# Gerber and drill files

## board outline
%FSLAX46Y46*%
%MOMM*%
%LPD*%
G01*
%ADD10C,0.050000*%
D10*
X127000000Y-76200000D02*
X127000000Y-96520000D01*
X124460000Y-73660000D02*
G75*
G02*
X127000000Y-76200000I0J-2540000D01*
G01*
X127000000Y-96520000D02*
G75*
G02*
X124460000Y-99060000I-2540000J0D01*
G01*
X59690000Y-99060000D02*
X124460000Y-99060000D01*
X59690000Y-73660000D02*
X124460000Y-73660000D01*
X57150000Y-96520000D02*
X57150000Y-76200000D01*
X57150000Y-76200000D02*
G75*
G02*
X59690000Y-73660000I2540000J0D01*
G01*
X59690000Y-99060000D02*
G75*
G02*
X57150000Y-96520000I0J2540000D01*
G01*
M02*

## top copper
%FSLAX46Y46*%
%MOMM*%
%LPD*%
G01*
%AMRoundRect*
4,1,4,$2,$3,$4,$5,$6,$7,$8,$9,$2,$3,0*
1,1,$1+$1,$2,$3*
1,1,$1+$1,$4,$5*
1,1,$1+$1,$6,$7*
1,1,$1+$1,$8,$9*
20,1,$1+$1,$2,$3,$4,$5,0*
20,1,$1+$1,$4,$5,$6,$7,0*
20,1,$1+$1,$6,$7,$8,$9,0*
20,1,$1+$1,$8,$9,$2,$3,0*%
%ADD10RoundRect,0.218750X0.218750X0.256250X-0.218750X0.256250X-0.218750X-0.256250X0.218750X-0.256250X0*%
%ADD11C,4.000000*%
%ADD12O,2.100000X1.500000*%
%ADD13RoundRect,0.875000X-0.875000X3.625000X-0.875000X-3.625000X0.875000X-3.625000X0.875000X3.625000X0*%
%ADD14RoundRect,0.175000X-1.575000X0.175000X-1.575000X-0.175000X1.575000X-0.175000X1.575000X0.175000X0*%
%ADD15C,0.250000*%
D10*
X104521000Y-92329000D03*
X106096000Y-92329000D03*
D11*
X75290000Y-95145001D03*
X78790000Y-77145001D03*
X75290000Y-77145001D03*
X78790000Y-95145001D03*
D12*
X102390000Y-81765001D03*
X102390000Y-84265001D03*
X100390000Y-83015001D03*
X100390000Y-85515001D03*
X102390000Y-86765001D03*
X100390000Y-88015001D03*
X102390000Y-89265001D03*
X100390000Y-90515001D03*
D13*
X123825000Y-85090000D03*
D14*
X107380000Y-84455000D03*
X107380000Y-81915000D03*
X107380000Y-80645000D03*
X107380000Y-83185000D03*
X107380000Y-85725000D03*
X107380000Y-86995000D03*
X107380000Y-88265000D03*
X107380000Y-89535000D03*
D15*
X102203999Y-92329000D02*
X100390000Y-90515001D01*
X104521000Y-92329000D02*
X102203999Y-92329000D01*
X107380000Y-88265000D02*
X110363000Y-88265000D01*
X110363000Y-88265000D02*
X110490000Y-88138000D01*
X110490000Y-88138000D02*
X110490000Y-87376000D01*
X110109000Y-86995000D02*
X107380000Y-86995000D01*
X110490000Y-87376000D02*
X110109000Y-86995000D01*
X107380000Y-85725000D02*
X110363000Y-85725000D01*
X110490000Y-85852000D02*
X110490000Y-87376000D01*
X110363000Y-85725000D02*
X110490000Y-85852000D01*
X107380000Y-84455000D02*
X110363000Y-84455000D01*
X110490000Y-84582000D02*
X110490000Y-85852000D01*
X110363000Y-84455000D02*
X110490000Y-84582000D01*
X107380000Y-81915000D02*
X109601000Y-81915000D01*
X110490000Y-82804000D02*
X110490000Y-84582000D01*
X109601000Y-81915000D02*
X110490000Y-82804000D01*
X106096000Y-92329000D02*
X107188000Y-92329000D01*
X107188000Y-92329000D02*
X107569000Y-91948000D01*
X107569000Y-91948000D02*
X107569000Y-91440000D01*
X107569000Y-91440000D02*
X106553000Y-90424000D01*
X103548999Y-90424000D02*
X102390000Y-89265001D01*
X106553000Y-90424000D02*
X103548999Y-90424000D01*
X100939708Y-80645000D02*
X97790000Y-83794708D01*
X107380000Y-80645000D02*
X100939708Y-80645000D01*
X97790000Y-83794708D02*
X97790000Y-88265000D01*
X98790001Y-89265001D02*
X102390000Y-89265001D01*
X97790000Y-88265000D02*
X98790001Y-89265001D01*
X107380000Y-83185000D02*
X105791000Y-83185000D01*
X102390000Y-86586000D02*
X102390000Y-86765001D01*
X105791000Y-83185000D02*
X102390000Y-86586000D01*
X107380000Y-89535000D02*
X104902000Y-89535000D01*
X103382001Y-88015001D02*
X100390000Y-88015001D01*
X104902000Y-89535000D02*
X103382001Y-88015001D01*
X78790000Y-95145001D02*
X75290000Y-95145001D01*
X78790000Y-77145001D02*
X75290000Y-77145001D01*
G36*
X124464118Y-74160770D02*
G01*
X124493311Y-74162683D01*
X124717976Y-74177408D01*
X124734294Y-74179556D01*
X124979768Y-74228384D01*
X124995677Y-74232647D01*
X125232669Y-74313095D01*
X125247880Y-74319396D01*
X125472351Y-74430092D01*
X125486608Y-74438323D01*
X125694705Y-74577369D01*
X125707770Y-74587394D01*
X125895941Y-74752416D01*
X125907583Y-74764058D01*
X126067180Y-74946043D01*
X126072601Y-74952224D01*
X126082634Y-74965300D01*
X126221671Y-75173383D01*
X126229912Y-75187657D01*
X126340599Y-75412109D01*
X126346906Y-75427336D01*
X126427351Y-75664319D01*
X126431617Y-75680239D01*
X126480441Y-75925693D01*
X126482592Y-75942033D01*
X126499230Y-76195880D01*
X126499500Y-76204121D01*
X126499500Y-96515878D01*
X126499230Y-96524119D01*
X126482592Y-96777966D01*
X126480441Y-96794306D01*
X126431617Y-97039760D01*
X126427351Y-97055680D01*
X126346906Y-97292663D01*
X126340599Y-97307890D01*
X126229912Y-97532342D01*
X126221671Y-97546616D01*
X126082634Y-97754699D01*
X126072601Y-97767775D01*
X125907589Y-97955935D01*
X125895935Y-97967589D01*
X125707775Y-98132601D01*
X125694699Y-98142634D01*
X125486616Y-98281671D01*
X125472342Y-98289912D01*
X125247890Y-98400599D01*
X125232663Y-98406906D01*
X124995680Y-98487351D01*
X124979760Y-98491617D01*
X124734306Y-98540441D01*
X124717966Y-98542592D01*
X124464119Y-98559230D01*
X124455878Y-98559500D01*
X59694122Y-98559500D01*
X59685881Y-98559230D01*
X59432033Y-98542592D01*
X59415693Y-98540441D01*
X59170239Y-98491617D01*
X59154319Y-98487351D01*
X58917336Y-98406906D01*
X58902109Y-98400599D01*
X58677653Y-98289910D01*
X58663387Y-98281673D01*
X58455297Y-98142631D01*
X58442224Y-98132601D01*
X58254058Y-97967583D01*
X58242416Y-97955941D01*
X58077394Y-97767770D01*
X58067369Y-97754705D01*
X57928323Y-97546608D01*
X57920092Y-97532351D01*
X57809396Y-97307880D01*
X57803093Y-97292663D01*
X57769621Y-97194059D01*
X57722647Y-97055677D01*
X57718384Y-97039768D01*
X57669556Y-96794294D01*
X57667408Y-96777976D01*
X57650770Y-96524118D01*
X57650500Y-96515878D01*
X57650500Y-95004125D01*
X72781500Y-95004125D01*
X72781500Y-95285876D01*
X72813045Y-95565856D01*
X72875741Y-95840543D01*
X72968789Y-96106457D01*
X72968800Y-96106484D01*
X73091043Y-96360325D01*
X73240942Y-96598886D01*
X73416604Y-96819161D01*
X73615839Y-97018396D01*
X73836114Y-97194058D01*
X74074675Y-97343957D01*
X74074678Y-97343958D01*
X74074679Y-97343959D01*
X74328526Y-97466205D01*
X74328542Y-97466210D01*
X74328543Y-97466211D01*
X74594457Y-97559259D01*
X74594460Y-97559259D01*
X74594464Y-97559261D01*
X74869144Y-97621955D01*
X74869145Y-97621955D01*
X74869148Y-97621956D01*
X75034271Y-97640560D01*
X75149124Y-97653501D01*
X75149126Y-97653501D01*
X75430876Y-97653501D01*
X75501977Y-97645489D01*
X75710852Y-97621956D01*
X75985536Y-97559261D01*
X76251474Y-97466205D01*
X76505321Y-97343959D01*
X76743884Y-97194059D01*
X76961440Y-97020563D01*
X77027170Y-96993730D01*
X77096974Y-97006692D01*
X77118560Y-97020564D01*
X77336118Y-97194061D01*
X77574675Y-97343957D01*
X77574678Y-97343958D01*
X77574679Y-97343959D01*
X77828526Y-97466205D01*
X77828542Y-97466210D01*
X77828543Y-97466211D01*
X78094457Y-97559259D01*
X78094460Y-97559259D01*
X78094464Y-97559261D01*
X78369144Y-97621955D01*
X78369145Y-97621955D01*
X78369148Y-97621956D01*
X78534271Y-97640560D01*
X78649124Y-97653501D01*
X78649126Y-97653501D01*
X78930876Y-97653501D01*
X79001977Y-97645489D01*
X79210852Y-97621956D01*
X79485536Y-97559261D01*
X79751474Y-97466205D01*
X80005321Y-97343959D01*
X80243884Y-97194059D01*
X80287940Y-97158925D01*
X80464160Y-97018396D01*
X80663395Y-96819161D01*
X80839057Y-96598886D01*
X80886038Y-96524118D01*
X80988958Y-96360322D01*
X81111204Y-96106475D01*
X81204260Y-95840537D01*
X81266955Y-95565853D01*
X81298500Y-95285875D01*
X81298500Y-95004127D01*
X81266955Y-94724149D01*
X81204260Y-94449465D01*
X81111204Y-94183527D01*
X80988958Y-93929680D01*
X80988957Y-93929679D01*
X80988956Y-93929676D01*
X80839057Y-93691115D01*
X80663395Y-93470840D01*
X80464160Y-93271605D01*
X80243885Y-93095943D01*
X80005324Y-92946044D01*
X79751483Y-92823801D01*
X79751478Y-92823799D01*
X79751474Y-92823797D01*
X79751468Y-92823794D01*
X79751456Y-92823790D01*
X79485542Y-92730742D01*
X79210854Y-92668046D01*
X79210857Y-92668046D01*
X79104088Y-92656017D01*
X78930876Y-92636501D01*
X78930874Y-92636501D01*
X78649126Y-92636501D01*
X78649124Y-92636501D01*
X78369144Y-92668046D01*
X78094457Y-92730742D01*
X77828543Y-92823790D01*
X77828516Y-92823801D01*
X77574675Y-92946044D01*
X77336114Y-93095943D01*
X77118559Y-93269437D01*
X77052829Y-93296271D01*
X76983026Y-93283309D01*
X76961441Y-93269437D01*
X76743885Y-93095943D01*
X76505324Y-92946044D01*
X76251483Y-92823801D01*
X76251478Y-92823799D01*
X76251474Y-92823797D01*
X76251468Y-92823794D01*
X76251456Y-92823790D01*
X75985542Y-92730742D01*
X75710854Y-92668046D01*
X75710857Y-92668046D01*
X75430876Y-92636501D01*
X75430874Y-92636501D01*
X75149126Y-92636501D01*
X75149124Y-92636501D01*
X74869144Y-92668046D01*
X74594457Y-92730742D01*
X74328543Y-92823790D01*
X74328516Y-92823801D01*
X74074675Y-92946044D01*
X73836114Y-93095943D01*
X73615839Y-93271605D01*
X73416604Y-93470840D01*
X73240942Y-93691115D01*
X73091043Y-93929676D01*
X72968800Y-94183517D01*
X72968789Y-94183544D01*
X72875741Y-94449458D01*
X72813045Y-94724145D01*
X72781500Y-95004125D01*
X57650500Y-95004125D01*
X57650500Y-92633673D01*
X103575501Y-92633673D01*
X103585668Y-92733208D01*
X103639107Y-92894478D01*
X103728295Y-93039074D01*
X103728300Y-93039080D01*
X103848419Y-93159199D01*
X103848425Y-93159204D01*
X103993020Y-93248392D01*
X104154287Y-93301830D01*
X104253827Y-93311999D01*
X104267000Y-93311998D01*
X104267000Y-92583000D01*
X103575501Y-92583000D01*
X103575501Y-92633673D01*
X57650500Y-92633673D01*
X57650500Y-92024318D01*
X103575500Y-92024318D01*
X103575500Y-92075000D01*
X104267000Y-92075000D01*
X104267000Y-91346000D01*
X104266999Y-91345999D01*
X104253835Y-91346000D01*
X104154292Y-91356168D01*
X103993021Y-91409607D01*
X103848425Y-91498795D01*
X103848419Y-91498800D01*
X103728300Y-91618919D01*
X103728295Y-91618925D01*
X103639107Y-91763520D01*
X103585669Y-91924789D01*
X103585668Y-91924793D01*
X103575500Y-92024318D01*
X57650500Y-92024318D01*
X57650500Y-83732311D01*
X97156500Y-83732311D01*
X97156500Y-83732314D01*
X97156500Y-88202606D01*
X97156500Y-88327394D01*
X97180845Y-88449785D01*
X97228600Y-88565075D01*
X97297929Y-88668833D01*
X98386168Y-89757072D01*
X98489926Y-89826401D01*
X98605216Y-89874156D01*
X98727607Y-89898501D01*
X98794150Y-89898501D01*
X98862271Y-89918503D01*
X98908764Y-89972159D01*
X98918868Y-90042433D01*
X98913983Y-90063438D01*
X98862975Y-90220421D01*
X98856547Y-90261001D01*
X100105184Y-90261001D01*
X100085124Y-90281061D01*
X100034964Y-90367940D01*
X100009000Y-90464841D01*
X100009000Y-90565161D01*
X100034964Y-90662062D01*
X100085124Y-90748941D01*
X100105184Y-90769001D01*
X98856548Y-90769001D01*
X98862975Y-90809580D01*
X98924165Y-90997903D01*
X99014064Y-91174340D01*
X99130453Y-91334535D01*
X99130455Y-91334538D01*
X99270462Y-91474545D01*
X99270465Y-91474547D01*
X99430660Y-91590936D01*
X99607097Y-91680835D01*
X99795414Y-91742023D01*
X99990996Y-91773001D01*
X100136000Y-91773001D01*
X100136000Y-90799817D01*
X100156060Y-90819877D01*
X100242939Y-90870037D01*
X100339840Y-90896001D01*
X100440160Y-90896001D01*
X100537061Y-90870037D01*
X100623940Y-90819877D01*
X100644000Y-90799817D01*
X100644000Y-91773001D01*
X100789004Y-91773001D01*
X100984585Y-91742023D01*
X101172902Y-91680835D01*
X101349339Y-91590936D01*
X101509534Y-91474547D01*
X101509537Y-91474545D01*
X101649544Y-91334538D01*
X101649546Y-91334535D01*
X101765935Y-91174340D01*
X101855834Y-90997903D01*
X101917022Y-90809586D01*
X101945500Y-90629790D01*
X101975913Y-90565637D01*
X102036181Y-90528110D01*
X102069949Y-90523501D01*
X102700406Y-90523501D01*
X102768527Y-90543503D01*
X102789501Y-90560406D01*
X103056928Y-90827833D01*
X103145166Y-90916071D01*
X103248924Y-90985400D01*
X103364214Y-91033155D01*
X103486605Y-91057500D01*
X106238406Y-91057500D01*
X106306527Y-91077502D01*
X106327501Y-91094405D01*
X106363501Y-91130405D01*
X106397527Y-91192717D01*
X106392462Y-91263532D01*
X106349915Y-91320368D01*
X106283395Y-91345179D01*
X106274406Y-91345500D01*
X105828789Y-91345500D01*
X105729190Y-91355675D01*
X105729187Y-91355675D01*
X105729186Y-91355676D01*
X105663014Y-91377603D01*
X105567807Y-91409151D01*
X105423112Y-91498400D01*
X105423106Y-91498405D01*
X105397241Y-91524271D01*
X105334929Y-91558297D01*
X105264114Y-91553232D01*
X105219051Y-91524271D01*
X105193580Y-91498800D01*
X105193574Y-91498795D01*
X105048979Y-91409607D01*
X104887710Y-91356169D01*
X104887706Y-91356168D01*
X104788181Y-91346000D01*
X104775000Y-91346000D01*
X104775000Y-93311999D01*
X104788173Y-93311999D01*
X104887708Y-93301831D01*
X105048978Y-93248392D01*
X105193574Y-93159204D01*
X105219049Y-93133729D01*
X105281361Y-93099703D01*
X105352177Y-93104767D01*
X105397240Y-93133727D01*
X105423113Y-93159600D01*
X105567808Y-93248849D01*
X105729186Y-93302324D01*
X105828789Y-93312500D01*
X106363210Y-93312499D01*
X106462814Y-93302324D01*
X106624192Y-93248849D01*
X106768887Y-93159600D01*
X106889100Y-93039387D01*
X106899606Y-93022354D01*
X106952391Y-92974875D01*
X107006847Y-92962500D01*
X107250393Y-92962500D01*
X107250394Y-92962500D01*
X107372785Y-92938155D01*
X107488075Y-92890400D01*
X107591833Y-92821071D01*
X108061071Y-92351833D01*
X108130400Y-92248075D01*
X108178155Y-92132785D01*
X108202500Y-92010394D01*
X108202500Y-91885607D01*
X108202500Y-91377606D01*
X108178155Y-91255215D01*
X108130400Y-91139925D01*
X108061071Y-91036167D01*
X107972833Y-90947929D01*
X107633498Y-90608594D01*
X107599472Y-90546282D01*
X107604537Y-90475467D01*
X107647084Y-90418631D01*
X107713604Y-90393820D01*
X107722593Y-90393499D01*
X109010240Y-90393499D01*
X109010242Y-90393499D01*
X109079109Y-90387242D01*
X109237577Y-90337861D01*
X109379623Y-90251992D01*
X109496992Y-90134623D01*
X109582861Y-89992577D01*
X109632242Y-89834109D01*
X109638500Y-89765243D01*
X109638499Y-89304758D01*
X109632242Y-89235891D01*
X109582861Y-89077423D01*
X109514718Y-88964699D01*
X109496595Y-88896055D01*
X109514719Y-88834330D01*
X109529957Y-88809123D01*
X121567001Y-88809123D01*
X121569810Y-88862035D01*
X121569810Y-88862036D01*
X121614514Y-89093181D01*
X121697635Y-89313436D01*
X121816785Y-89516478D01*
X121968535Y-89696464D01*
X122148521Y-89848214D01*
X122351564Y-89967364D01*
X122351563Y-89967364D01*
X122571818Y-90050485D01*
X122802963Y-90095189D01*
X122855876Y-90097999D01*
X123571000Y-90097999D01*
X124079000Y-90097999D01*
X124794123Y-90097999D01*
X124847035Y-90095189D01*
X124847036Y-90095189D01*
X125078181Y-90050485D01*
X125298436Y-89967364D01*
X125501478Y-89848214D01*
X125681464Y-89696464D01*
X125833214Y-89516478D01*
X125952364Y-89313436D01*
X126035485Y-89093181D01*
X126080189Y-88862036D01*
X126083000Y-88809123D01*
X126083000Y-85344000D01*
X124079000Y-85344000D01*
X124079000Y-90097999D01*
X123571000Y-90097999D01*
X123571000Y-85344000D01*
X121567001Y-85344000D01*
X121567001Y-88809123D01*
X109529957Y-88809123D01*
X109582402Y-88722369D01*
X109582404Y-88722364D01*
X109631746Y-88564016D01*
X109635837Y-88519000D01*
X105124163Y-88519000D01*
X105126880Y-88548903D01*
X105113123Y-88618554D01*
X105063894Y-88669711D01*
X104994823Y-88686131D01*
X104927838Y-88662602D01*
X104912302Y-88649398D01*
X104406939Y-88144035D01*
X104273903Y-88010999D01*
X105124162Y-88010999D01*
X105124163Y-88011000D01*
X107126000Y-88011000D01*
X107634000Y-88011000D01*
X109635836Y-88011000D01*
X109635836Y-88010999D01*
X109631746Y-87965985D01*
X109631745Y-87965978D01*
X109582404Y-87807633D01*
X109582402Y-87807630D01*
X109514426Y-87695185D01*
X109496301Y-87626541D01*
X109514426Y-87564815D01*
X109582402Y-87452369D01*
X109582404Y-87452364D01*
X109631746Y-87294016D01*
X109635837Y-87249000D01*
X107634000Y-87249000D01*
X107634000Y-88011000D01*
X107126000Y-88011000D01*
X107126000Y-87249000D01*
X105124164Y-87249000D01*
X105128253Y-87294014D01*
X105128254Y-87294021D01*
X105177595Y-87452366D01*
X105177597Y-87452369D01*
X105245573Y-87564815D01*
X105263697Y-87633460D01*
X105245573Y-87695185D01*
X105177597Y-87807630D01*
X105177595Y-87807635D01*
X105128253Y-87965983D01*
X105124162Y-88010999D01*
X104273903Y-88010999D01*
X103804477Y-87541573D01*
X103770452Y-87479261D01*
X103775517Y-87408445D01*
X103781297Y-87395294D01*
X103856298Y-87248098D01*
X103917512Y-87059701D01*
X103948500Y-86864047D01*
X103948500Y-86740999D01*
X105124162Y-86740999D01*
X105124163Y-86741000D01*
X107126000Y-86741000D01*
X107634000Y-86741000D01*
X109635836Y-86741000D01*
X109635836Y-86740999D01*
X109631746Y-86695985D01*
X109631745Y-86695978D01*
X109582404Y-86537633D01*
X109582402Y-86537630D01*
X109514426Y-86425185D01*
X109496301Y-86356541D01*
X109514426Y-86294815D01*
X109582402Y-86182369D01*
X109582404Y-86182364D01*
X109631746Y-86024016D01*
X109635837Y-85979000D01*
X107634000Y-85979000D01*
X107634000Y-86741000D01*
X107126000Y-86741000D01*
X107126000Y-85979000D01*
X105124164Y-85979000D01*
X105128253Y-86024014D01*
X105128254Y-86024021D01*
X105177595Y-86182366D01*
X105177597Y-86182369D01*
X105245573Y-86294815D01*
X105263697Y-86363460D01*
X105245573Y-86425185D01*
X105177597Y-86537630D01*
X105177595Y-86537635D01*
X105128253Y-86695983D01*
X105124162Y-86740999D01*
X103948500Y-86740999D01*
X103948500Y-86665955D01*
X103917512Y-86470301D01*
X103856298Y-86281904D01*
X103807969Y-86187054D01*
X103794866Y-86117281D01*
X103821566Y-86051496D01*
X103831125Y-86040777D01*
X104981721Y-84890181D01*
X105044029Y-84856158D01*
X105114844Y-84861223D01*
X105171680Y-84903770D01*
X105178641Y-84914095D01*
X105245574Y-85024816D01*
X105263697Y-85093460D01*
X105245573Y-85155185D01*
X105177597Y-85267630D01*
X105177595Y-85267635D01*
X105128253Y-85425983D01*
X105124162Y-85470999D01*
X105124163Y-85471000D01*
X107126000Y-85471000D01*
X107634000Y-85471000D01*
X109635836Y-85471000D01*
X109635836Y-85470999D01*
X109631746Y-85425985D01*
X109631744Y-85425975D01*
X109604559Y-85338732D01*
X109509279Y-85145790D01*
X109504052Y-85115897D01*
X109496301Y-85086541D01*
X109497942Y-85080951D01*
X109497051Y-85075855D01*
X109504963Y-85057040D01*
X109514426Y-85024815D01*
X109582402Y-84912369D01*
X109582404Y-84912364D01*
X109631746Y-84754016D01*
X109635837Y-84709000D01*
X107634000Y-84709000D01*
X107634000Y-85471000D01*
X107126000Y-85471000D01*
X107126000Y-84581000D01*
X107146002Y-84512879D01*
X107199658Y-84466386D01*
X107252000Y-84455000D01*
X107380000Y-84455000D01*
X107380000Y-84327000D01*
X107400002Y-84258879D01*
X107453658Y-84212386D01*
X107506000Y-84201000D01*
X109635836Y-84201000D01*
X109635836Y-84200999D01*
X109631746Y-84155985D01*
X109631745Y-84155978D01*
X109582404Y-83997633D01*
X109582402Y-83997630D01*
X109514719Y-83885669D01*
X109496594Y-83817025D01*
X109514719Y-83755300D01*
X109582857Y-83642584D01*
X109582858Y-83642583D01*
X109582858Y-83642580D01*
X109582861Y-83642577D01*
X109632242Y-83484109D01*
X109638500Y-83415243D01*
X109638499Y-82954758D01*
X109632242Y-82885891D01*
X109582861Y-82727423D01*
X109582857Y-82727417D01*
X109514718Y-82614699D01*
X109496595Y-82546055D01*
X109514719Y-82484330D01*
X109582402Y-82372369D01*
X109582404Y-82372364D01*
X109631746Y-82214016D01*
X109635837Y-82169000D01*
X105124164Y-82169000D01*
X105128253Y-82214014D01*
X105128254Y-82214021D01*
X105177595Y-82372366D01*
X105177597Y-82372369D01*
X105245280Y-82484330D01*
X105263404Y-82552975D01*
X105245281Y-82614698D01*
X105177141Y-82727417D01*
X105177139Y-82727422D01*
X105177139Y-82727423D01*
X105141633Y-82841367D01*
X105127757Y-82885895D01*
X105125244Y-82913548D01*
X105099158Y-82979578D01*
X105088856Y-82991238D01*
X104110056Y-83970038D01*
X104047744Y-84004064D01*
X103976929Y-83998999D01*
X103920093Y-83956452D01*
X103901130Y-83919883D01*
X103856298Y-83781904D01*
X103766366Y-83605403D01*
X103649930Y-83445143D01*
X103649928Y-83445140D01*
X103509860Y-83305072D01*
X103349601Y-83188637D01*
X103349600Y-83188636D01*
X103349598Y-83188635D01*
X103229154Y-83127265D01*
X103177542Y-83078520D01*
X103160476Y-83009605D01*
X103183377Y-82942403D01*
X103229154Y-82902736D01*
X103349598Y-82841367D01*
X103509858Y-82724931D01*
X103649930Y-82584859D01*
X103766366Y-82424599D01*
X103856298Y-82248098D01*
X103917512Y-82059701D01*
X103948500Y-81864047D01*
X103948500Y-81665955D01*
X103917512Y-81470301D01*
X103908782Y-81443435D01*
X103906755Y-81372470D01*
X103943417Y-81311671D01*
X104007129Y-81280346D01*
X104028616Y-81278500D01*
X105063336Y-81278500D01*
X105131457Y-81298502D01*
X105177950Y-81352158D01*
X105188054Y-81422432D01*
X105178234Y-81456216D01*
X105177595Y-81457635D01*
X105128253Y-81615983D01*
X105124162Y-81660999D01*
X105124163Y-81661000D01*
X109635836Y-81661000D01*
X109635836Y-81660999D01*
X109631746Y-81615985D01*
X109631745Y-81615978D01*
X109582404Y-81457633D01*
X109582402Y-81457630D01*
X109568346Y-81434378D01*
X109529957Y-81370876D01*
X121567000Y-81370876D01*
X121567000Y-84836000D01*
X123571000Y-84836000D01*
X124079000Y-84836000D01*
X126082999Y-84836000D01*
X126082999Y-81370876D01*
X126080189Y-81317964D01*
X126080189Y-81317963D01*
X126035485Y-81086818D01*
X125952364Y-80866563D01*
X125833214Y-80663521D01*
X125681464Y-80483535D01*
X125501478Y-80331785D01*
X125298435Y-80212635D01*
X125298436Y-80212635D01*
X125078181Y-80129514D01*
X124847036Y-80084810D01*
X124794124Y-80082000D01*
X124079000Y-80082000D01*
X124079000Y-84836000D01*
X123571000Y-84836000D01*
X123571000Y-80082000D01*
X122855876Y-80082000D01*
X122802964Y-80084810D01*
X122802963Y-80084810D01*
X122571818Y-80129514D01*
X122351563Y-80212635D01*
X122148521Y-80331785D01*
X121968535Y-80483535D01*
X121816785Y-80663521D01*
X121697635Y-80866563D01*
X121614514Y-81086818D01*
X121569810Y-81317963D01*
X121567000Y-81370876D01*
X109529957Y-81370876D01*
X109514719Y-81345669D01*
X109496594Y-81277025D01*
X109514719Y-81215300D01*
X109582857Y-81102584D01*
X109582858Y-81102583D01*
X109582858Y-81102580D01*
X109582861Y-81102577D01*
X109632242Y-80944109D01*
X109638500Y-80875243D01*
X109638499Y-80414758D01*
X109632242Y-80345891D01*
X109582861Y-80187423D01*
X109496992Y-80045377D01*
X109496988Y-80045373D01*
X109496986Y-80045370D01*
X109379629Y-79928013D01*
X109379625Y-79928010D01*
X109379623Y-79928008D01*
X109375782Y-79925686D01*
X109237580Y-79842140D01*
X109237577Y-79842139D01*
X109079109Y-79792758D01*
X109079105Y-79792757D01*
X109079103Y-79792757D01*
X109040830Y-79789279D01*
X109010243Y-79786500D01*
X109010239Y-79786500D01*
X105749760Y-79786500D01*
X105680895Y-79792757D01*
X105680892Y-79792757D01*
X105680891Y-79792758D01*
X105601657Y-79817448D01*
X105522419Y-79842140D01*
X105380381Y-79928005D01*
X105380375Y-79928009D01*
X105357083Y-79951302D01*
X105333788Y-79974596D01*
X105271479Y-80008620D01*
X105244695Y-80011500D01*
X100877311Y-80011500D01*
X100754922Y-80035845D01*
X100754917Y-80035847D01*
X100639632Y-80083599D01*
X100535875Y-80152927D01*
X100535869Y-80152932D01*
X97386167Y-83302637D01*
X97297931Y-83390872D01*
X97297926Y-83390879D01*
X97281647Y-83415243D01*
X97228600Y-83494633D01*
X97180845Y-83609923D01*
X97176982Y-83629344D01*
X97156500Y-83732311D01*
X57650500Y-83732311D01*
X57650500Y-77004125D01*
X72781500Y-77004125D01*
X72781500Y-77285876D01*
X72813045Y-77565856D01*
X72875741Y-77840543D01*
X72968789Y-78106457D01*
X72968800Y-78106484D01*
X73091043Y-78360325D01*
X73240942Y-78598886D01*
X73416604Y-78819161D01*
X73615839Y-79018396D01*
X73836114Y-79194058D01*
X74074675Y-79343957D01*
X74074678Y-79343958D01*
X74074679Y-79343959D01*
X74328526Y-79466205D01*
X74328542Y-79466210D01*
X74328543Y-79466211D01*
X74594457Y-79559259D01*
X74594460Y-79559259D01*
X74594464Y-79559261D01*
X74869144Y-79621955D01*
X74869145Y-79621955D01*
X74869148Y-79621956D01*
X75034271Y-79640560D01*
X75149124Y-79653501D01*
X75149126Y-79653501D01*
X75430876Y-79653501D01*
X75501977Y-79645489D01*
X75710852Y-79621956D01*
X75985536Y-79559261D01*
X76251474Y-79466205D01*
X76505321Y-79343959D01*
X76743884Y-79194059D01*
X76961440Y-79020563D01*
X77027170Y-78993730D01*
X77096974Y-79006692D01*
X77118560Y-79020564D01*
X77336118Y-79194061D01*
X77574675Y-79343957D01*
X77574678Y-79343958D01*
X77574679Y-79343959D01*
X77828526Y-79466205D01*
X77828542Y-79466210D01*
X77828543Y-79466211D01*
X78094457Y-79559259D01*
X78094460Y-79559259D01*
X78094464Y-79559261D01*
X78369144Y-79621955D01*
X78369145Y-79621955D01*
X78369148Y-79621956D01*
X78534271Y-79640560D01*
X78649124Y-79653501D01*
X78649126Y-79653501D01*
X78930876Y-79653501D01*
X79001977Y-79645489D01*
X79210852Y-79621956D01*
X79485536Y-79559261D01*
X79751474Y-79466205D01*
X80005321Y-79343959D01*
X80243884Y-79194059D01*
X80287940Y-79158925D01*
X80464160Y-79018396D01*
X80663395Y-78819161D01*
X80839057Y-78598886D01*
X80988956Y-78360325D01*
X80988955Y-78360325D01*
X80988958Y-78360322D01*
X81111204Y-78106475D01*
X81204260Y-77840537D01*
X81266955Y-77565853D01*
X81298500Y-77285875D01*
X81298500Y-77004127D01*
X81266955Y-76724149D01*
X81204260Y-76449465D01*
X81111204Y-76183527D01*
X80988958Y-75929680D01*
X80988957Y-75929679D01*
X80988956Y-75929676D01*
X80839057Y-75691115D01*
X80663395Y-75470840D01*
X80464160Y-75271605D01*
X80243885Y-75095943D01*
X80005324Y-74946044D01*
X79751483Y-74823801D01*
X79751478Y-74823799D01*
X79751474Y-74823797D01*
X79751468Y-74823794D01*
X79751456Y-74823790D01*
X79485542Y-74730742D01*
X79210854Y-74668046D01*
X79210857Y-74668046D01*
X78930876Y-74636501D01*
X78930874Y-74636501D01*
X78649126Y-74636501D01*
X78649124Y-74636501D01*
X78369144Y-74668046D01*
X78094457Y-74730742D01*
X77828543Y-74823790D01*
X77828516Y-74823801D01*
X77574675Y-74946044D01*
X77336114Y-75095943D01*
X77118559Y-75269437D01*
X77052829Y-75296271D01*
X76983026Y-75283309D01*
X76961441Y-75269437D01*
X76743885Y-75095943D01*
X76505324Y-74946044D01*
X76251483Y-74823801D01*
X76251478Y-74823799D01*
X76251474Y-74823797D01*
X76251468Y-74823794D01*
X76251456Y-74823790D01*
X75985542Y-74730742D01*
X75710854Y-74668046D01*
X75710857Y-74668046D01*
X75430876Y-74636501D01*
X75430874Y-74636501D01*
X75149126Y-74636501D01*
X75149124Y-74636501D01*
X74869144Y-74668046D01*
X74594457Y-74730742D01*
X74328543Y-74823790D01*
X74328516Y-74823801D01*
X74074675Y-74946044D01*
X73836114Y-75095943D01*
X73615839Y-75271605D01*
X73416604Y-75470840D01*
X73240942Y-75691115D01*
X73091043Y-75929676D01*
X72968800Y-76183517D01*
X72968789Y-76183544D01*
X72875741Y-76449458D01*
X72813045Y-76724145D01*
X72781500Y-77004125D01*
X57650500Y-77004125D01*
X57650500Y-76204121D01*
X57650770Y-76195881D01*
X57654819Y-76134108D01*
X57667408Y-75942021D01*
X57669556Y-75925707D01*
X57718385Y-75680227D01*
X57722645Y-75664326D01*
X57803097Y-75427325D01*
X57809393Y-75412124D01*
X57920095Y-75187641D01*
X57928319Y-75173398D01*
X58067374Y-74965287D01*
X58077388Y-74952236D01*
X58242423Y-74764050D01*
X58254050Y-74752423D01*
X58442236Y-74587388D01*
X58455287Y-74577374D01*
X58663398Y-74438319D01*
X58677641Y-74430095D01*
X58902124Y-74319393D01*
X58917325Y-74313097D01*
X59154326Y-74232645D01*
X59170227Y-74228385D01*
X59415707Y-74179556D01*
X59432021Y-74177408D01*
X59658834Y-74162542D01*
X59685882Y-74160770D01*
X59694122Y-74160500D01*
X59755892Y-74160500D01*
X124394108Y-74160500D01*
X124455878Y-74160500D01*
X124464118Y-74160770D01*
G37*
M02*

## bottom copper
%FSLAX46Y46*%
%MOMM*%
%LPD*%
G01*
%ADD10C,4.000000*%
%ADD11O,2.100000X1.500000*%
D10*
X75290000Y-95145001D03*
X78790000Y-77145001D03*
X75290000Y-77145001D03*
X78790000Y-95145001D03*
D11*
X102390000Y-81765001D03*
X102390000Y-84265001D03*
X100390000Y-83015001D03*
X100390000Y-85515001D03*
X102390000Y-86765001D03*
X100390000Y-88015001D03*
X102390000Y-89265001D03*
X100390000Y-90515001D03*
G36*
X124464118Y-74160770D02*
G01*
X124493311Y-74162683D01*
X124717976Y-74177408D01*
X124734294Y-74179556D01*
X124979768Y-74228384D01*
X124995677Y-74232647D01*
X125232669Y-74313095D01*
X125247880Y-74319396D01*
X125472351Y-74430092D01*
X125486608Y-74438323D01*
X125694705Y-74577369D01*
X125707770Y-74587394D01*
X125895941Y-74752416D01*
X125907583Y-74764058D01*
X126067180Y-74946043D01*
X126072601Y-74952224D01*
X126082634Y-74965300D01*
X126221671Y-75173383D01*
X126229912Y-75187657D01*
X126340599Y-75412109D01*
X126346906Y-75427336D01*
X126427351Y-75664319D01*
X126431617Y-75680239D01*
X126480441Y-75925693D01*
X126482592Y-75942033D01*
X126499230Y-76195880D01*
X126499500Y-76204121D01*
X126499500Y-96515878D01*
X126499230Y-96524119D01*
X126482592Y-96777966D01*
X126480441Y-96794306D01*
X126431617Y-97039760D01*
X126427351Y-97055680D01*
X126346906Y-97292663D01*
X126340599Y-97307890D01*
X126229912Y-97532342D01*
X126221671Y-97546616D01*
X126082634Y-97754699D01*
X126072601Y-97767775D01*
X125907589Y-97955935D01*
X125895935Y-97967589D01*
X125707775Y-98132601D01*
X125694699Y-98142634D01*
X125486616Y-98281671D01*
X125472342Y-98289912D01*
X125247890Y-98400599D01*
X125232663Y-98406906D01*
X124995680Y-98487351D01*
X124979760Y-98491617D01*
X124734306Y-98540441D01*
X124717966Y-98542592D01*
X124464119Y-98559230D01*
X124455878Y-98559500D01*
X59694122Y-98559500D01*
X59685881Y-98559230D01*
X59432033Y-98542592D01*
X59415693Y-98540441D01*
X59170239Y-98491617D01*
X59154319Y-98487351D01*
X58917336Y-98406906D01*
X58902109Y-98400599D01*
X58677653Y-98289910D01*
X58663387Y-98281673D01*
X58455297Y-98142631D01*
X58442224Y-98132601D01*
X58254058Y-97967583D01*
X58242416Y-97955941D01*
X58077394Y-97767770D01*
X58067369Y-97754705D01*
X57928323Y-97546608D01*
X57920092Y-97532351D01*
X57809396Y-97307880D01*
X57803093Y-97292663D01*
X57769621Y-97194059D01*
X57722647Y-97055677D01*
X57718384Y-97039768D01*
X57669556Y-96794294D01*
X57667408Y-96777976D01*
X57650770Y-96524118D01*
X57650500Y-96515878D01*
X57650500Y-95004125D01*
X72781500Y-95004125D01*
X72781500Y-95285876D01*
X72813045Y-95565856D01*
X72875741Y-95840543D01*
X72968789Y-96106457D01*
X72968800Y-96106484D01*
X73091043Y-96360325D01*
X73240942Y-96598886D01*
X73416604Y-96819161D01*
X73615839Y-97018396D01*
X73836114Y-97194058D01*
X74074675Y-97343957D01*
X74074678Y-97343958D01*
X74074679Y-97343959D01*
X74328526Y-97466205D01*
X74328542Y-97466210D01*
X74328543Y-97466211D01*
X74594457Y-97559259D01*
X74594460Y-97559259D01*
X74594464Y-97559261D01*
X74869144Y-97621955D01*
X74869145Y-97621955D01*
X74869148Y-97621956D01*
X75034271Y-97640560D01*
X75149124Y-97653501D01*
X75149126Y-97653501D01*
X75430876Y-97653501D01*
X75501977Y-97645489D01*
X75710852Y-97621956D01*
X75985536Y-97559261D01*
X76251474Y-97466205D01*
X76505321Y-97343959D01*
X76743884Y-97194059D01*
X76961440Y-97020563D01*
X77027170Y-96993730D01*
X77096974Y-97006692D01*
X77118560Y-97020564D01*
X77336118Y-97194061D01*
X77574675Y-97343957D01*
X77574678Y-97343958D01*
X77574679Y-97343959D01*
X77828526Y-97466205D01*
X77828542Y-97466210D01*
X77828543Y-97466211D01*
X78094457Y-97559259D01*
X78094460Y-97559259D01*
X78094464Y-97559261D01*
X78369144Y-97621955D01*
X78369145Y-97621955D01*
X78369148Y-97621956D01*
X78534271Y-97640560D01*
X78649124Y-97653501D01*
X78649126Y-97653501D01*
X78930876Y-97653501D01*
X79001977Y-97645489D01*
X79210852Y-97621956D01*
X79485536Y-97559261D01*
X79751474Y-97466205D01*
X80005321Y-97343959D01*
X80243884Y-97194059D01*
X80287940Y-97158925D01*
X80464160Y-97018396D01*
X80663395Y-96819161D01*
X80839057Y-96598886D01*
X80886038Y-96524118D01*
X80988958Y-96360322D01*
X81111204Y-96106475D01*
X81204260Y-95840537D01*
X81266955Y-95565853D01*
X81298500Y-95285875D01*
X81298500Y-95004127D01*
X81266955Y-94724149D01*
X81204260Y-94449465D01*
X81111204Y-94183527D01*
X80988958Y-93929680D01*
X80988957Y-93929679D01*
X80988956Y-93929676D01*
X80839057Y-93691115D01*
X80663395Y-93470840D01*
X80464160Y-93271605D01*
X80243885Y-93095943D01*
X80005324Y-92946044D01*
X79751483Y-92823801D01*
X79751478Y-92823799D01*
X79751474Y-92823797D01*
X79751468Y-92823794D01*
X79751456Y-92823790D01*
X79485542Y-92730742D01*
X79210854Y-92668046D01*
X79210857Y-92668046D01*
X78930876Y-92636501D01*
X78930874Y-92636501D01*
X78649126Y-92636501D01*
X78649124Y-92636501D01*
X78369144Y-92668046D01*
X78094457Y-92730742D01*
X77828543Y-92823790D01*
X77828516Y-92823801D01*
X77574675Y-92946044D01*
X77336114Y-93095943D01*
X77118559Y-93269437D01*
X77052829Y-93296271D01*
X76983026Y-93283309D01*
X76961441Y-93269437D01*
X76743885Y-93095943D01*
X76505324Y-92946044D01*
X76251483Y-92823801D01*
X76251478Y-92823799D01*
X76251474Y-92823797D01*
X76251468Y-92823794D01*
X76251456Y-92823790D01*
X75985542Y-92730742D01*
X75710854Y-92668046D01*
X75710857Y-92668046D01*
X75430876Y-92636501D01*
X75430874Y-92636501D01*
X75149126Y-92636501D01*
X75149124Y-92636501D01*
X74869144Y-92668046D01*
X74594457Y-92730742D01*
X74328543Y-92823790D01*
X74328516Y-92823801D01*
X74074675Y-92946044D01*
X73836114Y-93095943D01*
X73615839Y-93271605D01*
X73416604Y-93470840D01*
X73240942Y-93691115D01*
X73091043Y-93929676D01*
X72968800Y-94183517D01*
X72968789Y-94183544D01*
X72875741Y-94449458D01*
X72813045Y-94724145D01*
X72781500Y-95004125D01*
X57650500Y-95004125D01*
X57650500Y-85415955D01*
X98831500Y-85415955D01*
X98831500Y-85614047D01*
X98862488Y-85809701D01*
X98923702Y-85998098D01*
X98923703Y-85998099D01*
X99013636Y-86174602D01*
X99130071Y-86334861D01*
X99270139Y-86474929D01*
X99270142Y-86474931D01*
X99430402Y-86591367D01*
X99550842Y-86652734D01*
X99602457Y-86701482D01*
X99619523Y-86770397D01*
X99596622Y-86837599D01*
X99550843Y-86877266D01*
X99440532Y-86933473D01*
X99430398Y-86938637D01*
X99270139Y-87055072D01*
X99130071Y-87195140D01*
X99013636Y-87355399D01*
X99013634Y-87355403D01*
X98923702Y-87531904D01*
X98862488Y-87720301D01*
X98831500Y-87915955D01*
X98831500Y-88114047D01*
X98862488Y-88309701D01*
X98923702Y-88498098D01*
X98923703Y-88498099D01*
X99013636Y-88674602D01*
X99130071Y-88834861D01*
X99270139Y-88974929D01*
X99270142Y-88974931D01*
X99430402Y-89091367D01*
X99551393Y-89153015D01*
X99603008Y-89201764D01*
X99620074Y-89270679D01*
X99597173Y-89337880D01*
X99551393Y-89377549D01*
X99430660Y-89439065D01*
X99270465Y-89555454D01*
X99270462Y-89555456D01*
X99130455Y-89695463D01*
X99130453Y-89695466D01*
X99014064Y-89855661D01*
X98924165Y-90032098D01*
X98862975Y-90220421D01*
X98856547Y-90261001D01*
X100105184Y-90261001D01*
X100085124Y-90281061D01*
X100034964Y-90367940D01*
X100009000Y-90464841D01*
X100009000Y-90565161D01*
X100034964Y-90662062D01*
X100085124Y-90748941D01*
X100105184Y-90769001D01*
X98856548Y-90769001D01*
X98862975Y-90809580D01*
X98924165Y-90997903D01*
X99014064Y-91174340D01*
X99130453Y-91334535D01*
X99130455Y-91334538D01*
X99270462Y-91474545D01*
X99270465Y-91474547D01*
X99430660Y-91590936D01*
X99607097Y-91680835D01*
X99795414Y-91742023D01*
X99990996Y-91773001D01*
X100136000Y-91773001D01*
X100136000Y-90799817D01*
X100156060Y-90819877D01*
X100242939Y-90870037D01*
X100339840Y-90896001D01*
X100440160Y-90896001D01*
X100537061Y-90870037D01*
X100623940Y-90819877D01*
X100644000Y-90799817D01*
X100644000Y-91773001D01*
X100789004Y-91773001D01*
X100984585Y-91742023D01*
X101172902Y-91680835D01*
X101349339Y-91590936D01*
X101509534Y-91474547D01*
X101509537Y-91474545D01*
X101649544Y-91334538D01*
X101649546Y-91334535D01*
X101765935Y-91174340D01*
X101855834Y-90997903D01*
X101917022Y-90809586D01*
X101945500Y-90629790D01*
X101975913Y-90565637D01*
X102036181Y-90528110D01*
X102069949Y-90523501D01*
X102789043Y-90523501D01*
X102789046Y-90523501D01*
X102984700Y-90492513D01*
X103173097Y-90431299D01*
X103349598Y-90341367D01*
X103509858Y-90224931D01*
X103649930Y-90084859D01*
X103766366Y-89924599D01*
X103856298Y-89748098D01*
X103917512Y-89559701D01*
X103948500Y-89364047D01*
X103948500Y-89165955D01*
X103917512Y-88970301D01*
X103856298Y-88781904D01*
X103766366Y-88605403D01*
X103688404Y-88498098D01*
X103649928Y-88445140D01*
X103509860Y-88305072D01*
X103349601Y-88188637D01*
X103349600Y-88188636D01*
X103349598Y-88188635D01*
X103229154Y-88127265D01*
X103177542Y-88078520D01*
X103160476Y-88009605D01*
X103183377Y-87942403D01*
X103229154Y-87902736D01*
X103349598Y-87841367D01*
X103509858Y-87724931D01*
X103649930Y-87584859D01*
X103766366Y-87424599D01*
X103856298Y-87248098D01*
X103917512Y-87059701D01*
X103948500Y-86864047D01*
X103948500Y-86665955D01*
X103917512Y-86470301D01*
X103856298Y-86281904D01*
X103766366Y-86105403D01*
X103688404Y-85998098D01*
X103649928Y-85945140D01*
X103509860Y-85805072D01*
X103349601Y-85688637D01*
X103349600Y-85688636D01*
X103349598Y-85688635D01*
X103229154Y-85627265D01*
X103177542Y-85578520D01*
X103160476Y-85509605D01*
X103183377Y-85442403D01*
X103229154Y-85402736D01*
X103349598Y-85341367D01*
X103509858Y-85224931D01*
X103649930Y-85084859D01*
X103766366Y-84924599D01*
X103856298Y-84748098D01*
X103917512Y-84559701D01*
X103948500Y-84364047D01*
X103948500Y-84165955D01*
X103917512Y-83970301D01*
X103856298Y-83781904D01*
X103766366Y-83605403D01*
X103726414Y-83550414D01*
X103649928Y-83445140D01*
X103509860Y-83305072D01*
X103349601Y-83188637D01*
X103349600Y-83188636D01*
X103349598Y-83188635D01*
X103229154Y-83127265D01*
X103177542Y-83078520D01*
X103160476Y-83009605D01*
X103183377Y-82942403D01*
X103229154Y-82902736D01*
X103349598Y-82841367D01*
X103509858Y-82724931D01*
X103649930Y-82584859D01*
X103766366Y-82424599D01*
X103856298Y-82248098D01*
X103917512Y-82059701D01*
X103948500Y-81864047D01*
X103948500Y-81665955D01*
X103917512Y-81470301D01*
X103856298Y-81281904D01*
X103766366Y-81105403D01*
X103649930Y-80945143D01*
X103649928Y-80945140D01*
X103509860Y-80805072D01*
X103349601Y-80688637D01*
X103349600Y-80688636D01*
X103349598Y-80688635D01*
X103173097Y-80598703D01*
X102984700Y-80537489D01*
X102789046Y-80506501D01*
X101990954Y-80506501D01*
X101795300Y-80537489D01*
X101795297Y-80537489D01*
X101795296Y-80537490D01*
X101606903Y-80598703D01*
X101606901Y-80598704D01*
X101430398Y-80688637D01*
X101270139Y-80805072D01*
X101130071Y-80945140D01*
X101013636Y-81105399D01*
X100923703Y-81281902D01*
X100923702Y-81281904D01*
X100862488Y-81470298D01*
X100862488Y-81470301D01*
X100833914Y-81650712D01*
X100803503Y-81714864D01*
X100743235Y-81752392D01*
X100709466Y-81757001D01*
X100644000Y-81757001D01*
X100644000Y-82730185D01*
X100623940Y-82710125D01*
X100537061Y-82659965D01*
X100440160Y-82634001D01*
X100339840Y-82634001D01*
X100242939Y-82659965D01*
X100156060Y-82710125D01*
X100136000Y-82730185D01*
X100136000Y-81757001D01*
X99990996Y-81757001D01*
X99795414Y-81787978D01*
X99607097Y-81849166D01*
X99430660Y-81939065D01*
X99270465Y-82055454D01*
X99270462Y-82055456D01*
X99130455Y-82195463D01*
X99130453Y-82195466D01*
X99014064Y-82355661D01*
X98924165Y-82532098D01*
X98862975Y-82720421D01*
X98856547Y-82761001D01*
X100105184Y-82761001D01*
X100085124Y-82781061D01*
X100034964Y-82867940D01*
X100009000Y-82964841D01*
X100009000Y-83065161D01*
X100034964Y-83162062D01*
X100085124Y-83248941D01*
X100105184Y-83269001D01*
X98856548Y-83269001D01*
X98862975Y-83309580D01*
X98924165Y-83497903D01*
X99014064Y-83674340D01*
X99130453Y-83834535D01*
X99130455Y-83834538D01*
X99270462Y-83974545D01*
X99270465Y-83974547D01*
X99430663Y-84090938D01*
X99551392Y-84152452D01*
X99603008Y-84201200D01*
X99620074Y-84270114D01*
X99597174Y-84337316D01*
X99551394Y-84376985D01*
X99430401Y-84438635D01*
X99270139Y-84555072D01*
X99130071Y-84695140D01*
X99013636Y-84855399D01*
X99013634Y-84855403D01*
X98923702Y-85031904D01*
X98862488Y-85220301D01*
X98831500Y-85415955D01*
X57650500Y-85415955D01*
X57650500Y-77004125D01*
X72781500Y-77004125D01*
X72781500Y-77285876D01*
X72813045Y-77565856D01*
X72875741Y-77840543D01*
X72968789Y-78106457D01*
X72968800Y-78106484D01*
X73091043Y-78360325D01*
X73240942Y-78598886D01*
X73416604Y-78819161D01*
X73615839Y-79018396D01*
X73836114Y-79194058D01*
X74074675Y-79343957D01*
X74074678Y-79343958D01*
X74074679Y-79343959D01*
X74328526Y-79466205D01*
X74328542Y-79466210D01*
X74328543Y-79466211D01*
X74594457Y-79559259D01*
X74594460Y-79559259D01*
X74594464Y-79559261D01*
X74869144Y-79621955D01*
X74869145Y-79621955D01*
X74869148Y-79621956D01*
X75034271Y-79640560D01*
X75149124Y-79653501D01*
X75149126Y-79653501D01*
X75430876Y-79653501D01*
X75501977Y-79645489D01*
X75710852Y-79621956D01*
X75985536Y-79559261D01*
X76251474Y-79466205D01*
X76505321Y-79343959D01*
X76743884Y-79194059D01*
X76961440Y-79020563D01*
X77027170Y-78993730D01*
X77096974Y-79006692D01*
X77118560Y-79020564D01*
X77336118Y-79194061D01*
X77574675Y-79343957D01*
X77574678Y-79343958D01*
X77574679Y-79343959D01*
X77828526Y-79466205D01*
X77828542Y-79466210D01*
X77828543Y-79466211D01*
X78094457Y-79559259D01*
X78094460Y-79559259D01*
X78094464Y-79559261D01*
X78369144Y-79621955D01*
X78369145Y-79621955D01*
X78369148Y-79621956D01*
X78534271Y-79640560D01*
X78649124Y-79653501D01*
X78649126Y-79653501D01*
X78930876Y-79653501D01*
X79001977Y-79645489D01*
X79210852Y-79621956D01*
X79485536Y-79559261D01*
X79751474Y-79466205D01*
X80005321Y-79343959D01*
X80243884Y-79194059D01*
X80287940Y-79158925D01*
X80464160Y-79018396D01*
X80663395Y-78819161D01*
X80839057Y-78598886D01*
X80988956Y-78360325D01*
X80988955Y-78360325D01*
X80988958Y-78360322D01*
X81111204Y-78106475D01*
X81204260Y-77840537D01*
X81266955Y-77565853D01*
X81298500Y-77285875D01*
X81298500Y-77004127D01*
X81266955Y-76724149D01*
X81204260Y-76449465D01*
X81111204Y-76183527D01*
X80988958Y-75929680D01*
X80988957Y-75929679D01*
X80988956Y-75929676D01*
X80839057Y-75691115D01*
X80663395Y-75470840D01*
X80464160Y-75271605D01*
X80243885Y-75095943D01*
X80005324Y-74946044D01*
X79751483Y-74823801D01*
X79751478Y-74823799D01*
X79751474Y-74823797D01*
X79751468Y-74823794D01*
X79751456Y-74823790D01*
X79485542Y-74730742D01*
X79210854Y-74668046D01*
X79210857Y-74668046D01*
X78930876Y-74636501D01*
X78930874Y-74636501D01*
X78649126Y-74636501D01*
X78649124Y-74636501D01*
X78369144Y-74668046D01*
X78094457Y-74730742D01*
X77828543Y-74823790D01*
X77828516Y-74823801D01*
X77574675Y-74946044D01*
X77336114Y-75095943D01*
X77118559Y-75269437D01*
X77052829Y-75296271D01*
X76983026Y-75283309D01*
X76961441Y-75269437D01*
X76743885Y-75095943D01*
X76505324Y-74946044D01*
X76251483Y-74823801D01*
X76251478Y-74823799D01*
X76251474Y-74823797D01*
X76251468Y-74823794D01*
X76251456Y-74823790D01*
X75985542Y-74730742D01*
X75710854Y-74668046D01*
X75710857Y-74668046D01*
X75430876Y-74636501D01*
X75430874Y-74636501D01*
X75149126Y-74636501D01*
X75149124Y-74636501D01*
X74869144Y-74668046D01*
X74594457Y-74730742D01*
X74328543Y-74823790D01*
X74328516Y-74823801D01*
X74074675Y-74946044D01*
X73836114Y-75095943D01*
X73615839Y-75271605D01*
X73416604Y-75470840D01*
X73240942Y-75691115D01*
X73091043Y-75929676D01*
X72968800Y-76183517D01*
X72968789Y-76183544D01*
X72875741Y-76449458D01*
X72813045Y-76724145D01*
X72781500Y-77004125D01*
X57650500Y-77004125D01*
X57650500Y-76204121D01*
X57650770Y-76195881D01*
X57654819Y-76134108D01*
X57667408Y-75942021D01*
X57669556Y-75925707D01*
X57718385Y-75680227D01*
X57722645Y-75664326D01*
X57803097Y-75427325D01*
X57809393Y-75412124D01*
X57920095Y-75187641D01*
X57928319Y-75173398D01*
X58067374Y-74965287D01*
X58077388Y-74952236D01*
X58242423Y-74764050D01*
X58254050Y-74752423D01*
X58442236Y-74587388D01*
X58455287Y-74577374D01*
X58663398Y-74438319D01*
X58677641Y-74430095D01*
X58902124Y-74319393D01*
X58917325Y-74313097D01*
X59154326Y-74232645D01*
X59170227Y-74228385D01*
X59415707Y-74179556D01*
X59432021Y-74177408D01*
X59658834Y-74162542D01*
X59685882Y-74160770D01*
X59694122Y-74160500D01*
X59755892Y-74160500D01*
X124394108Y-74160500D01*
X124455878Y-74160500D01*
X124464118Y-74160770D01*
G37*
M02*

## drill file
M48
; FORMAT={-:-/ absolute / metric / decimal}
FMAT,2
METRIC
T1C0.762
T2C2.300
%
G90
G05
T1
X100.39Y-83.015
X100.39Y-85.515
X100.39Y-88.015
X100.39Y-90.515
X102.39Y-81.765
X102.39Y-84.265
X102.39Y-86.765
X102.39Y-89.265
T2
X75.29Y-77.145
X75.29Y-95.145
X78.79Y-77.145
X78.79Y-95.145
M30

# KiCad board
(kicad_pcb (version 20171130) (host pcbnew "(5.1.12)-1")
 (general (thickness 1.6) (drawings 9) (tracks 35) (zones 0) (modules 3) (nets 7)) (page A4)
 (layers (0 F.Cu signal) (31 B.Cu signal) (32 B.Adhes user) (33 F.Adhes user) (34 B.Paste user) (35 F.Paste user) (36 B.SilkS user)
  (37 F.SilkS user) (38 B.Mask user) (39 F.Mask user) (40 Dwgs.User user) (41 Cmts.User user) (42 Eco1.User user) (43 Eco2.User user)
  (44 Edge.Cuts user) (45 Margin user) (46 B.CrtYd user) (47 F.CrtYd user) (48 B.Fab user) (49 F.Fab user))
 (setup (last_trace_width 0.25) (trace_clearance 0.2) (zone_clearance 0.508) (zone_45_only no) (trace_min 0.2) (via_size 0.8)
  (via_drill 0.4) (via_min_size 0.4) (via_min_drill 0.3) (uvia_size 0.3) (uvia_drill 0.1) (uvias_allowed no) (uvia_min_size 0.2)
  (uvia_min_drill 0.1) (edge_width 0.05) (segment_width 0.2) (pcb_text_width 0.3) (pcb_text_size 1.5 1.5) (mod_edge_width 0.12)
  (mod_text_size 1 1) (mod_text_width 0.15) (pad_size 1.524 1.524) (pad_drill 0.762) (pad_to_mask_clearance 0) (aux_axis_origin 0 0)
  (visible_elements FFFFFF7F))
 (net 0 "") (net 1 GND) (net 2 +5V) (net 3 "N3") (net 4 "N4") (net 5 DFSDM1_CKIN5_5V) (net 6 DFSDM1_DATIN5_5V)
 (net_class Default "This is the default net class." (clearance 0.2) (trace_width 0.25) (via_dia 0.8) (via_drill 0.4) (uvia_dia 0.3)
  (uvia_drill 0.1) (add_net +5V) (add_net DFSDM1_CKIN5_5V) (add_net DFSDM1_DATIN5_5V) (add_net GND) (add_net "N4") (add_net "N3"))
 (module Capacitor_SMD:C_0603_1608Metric (layer F.Cu) (at 105.3085 92.329 180)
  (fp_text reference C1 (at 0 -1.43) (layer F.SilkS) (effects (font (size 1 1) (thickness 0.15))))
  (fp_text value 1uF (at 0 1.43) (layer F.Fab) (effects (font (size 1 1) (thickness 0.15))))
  (pad 2 smd roundrect (at 0.7875 0 180) (size 0.875 0.95) (layers F.Cu F.Paste F.Mask) (roundrect_rratio 0.25) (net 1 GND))
  (pad 1 smd roundrect (at -0.7875 0 180) (size 0.875 0.95) (layers F.Cu F.Paste F.Mask) (roundrect_rratio 0.25) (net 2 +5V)))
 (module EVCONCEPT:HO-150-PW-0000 (layer F.Cu) (at 100.39 86.145001)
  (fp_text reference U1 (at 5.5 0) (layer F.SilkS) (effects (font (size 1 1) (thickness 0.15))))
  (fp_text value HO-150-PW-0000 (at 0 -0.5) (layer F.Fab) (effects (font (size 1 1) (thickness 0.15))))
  (pad 9 thru_hole circle (at -25.1 9) (size 4 4) (drill 2.3) (layers *.Cu *.Mask) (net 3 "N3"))
  (pad 10 thru_hole circle (at -21.6 -9) (size 4 4) (drill 2.3) (layers *.Cu *.Mask) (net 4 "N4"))
  (pad 10 thru_hole circle (at -25.1 -9) (size 4 4) (drill 2.3) (layers *.Cu *.Mask) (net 4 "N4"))
  (pad 9 thru_hole circle (at -21.6 9) (size 4 4) (drill 2.3) (layers *.Cu *.Mask) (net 3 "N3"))
  (pad 1 thru_hole oval (at 2 -4.38) (size 2.1 1.5) (drill 0.762) (layers *.Cu *.Mask))
  (pad 3 thru_hole oval (at 2 -1.88) (size 2.1 1.5) (drill 0.762) (layers *.Cu *.Mask))
  (pad 2 thru_hole oval (at 0 -3.13) (size 2.1 1.5) (drill 0.762) (layers *.Cu *.Mask) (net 1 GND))
  (pad 4 thru_hole oval (at 0 -0.63) (size 2.1 1.5) (drill 0.762) (layers *.Cu *.Mask))
  (pad 5 thru_hole oval (at 2 0.62) (size 2.1 1.5) (drill 0.762) (layers *.Cu *.Mask) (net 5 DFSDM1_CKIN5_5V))
  (pad 6 thru_hole oval (at 0 1.87) (size 2.1 1.5) (drill 0.762) (layers *.Cu *.Mask) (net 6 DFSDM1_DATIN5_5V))
  (pad 7 thru_hole oval (at 2 3.12) (size 2.1 1.5) (drill 0.762) (layers *.Cu *.Mask) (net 2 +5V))
  (pad 8 thru_hole oval (at 0 4.37) (size 2.1 1.5) (drill 0.762) (layers *.Cu *.Mask) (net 1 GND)))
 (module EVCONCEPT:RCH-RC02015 (layer F.Cu) (at 115.57 85.09 270)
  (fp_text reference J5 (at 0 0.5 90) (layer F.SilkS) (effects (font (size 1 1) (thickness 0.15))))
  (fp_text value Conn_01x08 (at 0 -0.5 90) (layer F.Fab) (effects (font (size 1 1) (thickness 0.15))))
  (pad 9 smd roundrect (at 0 -8.255 270) (size 9 3.5) (layers F.Cu F.Paste F.Mask) (roundrect_rratio 0.25) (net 1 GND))
  (pad 5 smd roundrect (at -0.635 8.19 270) (size 0.7 3.5) (layers F.Cu F.Paste F.Mask) (roundrect_rratio 0.25) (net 1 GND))
  (pad 7 smd roundrect (at -3.175 8.19 270) (size 0.7 3.5) (layers F.Cu F.Paste F.Mask) (roundrect_rratio 0.25) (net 1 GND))
  (pad 8 smd roundrect (at -4.445 8.19 270) (size 0.7 3.5) (layers F.Cu F.Paste F.Mask) (roundrect_rratio 0.25) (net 2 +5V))
  (pad 6 smd roundrect (at -1.905 8.19 270) (size 0.7 3.5) (layers F.Cu F.Paste F.Mask) (roundrect_rratio 0.25) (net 5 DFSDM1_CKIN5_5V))
  (pad 4 smd roundrect (at 0.635 8.19 270) (size 0.7 3.5) (layers F.Cu F.Paste F.Mask) (roundrect_rratio 0.25) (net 1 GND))
  (pad 3 smd roundrect (at 1.905 8.19 270) (size 0.7 3.5) (layers F.Cu F.Paste F.Mask) (roundrect_rratio 0.25) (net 1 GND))
  (pad 2 smd roundrect (at 3.175 8.19 270) (size 0.7 3.5) (layers F.Cu F.Paste F.Mask) (roundrect_rratio 0.25) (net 1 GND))
  (pad 1 smd roundrect (at 4.445 8.19 270) (size 0.7 3.5) (layers F.Cu F.Paste F.Mask) (roundrect_rratio 0.25) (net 6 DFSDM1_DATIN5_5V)))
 (gr_line (start 127 76.2) (end 127 96.52) (layer Edge.Cuts) (width 0.05))
 (gr_arc (start 124.46 76.2) (end 127 76.2) (angle -90) (layer Edge.Cuts) (width 0.05))
 (gr_arc (start 124.46 96.52) (end 124.46 99.06) (angle -90) (layer Edge.Cuts) (width 0.05))
 (gr_line (start 59.69 99.06) (end 124.46 99.06) (layer Edge.Cuts) (width 0.05))
 (gr_line (start 59.69 73.66) (end 124.46 73.66) (layer Edge.Cuts) (width 0.05))
 (gr_line (start 57.15 96.52) (end 57.15 76.2) (layer Edge.Cuts) (width 0.05))
 (gr_arc (start 59.69 76.2) (end 59.69 73.66) (angle -90) (layer Edge.Cuts) (width 0.05))
 (gr_arc (start 59.69 96.52) (end 57.15 96.52) (angle -90) (layer Edge.Cuts) (width 0.05))
 (segment (start 102.203999 92.329) (end 100.39 90.515001) (width 0.25) (layer F.Cu) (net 1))
 (segment (start 104.521 92.329) (end 102.203999 92.329) (width 0.25) (layer F.Cu) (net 1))
 (segment (start 107.38 88.265) (end 110.363 88.265) (width 0.25) (layer F.Cu) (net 1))
 (segment (start 110.363 88.265) (end 110.49 88.138) (width 0.25) (layer F.Cu) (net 1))
 (segment (start 110.49 88.138) (end 110.49 87.376) (width 0.25) (layer F.Cu) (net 1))
 (segment (start 110.109 86.995) (end 107.38 86.995) (width 0.25) (layer F.Cu) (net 1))
 (segment (start 110.49 87.376) (end 110.109 86.995) (width 0.25) (layer F.Cu) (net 1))
 (segment (start 107.38 85.725) (end 110.363 85.725) (width 0.25) (layer F.Cu) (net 1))
 (segment (start 110.49 85.852) (end 110.49 87.376) (width 0.25) (layer F.Cu) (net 1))
 (segment (start 110.363 85.725) (end 110.49 85.852) (width 0.25) (layer F.Cu) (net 1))
 (segment (start 107.38 84.455) (end 110.363 84.455) (width 0.25) (layer F.Cu) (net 1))
 (segment (start 110.49 84.582) (end 110.49 85.852) (width 0.25) (layer F.Cu) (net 1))
 (segment (start 110.363 84.455) (end 110.49 84.582) (width 0.25) (layer F.Cu) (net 1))
 (segment (start 107.38 81.915) (end 109.601 81.915) (width 0.25) (layer F.Cu) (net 1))
 (segment (start 110.49 82.804) (end 110.49 84.582) (width 0.25) (layer F.Cu) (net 1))
 (segment (start 109.601 81.915) (end 110.49 82.804) (width 0.25) (layer F.Cu) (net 1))
 (segment (start 106.096 92.329) (end 107.188 92.329) (width 0.25) (layer F.Cu) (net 2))
 (segment (start 107.188 92.329) (end 107.569 91.948) (width 0.25) (layer F.Cu) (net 2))
 (segment (start 107.569 91.948) (end 107.569 91.44) (width 0.25) (layer F.Cu) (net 2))
 (segment (start 107.569 91.44) (end 106.553 90.424) (width 0.25) (layer F.Cu) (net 2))
 (segment (start 103.548999 90.424) (end 102.39 89.265001) (width 0.25) (layer F.Cu) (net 2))
 (segment (start 106.553 90.424) (end 103.548999 90.424) (width 0.25) (layer F.Cu) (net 2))
 (segment (start 100.939708 80.645) (end 97.79 83.794708) (width 0.25) (layer F.Cu) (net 2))
 (segment (start 107.38 80.645) (end 100.939708 80.645) (width 0.25) (layer F.Cu) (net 2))
 (segment (start 97.79 83.794708) (end 97.79 88.265) (width 0.25) (layer F.Cu) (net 2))
 (segment (start 98.790001 89.265001) (end 102.39 89.265001) (width 0.25) (layer F.Cu) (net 2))
 (segment (start 97.79 88.265) (end 98.790001 89.265001) (width 0.25) (layer F.Cu) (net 2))
 (segment (start 107.38 83.185) (end 105.791 83.185) (width 0.25) (layer F.Cu) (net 5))
 (segment (start 102.39 86.586) (end 102.39 86.765001) (width 0.25) (layer F.Cu) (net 5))
 (segment (start 105.791 83.185) (end 102.39 86.586) (width 0.25) (layer F.Cu) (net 5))
 (segment (start 107.38 89.535) (end 104.902 89.535) (width 0.25) (layer F.Cu) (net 6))
 (segment (start 103.382001 88.015001) (end 100.39 88.015001) (width 0.25) (layer F.Cu) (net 6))
 (segment (start 104.902 89.535) (end 103.382001 88.015001) (width 0.25) (layer F.Cu) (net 6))
 (segment (start 78.79 95.145001) (end 75.29 95.145001) (width 0.25) (layer F.Cu) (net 3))
 (segment (start 78.79 77.145001) (end 75.29 77.145001) (width 0.25) (layer F.Cu) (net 4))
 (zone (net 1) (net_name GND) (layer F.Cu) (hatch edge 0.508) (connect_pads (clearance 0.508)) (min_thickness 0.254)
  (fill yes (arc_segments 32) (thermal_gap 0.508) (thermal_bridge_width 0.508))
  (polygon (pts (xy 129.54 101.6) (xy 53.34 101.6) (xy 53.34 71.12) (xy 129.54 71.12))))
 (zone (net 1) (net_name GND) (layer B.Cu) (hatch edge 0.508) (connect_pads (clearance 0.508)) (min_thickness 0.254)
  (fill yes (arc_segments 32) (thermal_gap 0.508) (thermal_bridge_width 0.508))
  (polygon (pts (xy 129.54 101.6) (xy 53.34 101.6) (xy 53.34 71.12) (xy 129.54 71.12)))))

